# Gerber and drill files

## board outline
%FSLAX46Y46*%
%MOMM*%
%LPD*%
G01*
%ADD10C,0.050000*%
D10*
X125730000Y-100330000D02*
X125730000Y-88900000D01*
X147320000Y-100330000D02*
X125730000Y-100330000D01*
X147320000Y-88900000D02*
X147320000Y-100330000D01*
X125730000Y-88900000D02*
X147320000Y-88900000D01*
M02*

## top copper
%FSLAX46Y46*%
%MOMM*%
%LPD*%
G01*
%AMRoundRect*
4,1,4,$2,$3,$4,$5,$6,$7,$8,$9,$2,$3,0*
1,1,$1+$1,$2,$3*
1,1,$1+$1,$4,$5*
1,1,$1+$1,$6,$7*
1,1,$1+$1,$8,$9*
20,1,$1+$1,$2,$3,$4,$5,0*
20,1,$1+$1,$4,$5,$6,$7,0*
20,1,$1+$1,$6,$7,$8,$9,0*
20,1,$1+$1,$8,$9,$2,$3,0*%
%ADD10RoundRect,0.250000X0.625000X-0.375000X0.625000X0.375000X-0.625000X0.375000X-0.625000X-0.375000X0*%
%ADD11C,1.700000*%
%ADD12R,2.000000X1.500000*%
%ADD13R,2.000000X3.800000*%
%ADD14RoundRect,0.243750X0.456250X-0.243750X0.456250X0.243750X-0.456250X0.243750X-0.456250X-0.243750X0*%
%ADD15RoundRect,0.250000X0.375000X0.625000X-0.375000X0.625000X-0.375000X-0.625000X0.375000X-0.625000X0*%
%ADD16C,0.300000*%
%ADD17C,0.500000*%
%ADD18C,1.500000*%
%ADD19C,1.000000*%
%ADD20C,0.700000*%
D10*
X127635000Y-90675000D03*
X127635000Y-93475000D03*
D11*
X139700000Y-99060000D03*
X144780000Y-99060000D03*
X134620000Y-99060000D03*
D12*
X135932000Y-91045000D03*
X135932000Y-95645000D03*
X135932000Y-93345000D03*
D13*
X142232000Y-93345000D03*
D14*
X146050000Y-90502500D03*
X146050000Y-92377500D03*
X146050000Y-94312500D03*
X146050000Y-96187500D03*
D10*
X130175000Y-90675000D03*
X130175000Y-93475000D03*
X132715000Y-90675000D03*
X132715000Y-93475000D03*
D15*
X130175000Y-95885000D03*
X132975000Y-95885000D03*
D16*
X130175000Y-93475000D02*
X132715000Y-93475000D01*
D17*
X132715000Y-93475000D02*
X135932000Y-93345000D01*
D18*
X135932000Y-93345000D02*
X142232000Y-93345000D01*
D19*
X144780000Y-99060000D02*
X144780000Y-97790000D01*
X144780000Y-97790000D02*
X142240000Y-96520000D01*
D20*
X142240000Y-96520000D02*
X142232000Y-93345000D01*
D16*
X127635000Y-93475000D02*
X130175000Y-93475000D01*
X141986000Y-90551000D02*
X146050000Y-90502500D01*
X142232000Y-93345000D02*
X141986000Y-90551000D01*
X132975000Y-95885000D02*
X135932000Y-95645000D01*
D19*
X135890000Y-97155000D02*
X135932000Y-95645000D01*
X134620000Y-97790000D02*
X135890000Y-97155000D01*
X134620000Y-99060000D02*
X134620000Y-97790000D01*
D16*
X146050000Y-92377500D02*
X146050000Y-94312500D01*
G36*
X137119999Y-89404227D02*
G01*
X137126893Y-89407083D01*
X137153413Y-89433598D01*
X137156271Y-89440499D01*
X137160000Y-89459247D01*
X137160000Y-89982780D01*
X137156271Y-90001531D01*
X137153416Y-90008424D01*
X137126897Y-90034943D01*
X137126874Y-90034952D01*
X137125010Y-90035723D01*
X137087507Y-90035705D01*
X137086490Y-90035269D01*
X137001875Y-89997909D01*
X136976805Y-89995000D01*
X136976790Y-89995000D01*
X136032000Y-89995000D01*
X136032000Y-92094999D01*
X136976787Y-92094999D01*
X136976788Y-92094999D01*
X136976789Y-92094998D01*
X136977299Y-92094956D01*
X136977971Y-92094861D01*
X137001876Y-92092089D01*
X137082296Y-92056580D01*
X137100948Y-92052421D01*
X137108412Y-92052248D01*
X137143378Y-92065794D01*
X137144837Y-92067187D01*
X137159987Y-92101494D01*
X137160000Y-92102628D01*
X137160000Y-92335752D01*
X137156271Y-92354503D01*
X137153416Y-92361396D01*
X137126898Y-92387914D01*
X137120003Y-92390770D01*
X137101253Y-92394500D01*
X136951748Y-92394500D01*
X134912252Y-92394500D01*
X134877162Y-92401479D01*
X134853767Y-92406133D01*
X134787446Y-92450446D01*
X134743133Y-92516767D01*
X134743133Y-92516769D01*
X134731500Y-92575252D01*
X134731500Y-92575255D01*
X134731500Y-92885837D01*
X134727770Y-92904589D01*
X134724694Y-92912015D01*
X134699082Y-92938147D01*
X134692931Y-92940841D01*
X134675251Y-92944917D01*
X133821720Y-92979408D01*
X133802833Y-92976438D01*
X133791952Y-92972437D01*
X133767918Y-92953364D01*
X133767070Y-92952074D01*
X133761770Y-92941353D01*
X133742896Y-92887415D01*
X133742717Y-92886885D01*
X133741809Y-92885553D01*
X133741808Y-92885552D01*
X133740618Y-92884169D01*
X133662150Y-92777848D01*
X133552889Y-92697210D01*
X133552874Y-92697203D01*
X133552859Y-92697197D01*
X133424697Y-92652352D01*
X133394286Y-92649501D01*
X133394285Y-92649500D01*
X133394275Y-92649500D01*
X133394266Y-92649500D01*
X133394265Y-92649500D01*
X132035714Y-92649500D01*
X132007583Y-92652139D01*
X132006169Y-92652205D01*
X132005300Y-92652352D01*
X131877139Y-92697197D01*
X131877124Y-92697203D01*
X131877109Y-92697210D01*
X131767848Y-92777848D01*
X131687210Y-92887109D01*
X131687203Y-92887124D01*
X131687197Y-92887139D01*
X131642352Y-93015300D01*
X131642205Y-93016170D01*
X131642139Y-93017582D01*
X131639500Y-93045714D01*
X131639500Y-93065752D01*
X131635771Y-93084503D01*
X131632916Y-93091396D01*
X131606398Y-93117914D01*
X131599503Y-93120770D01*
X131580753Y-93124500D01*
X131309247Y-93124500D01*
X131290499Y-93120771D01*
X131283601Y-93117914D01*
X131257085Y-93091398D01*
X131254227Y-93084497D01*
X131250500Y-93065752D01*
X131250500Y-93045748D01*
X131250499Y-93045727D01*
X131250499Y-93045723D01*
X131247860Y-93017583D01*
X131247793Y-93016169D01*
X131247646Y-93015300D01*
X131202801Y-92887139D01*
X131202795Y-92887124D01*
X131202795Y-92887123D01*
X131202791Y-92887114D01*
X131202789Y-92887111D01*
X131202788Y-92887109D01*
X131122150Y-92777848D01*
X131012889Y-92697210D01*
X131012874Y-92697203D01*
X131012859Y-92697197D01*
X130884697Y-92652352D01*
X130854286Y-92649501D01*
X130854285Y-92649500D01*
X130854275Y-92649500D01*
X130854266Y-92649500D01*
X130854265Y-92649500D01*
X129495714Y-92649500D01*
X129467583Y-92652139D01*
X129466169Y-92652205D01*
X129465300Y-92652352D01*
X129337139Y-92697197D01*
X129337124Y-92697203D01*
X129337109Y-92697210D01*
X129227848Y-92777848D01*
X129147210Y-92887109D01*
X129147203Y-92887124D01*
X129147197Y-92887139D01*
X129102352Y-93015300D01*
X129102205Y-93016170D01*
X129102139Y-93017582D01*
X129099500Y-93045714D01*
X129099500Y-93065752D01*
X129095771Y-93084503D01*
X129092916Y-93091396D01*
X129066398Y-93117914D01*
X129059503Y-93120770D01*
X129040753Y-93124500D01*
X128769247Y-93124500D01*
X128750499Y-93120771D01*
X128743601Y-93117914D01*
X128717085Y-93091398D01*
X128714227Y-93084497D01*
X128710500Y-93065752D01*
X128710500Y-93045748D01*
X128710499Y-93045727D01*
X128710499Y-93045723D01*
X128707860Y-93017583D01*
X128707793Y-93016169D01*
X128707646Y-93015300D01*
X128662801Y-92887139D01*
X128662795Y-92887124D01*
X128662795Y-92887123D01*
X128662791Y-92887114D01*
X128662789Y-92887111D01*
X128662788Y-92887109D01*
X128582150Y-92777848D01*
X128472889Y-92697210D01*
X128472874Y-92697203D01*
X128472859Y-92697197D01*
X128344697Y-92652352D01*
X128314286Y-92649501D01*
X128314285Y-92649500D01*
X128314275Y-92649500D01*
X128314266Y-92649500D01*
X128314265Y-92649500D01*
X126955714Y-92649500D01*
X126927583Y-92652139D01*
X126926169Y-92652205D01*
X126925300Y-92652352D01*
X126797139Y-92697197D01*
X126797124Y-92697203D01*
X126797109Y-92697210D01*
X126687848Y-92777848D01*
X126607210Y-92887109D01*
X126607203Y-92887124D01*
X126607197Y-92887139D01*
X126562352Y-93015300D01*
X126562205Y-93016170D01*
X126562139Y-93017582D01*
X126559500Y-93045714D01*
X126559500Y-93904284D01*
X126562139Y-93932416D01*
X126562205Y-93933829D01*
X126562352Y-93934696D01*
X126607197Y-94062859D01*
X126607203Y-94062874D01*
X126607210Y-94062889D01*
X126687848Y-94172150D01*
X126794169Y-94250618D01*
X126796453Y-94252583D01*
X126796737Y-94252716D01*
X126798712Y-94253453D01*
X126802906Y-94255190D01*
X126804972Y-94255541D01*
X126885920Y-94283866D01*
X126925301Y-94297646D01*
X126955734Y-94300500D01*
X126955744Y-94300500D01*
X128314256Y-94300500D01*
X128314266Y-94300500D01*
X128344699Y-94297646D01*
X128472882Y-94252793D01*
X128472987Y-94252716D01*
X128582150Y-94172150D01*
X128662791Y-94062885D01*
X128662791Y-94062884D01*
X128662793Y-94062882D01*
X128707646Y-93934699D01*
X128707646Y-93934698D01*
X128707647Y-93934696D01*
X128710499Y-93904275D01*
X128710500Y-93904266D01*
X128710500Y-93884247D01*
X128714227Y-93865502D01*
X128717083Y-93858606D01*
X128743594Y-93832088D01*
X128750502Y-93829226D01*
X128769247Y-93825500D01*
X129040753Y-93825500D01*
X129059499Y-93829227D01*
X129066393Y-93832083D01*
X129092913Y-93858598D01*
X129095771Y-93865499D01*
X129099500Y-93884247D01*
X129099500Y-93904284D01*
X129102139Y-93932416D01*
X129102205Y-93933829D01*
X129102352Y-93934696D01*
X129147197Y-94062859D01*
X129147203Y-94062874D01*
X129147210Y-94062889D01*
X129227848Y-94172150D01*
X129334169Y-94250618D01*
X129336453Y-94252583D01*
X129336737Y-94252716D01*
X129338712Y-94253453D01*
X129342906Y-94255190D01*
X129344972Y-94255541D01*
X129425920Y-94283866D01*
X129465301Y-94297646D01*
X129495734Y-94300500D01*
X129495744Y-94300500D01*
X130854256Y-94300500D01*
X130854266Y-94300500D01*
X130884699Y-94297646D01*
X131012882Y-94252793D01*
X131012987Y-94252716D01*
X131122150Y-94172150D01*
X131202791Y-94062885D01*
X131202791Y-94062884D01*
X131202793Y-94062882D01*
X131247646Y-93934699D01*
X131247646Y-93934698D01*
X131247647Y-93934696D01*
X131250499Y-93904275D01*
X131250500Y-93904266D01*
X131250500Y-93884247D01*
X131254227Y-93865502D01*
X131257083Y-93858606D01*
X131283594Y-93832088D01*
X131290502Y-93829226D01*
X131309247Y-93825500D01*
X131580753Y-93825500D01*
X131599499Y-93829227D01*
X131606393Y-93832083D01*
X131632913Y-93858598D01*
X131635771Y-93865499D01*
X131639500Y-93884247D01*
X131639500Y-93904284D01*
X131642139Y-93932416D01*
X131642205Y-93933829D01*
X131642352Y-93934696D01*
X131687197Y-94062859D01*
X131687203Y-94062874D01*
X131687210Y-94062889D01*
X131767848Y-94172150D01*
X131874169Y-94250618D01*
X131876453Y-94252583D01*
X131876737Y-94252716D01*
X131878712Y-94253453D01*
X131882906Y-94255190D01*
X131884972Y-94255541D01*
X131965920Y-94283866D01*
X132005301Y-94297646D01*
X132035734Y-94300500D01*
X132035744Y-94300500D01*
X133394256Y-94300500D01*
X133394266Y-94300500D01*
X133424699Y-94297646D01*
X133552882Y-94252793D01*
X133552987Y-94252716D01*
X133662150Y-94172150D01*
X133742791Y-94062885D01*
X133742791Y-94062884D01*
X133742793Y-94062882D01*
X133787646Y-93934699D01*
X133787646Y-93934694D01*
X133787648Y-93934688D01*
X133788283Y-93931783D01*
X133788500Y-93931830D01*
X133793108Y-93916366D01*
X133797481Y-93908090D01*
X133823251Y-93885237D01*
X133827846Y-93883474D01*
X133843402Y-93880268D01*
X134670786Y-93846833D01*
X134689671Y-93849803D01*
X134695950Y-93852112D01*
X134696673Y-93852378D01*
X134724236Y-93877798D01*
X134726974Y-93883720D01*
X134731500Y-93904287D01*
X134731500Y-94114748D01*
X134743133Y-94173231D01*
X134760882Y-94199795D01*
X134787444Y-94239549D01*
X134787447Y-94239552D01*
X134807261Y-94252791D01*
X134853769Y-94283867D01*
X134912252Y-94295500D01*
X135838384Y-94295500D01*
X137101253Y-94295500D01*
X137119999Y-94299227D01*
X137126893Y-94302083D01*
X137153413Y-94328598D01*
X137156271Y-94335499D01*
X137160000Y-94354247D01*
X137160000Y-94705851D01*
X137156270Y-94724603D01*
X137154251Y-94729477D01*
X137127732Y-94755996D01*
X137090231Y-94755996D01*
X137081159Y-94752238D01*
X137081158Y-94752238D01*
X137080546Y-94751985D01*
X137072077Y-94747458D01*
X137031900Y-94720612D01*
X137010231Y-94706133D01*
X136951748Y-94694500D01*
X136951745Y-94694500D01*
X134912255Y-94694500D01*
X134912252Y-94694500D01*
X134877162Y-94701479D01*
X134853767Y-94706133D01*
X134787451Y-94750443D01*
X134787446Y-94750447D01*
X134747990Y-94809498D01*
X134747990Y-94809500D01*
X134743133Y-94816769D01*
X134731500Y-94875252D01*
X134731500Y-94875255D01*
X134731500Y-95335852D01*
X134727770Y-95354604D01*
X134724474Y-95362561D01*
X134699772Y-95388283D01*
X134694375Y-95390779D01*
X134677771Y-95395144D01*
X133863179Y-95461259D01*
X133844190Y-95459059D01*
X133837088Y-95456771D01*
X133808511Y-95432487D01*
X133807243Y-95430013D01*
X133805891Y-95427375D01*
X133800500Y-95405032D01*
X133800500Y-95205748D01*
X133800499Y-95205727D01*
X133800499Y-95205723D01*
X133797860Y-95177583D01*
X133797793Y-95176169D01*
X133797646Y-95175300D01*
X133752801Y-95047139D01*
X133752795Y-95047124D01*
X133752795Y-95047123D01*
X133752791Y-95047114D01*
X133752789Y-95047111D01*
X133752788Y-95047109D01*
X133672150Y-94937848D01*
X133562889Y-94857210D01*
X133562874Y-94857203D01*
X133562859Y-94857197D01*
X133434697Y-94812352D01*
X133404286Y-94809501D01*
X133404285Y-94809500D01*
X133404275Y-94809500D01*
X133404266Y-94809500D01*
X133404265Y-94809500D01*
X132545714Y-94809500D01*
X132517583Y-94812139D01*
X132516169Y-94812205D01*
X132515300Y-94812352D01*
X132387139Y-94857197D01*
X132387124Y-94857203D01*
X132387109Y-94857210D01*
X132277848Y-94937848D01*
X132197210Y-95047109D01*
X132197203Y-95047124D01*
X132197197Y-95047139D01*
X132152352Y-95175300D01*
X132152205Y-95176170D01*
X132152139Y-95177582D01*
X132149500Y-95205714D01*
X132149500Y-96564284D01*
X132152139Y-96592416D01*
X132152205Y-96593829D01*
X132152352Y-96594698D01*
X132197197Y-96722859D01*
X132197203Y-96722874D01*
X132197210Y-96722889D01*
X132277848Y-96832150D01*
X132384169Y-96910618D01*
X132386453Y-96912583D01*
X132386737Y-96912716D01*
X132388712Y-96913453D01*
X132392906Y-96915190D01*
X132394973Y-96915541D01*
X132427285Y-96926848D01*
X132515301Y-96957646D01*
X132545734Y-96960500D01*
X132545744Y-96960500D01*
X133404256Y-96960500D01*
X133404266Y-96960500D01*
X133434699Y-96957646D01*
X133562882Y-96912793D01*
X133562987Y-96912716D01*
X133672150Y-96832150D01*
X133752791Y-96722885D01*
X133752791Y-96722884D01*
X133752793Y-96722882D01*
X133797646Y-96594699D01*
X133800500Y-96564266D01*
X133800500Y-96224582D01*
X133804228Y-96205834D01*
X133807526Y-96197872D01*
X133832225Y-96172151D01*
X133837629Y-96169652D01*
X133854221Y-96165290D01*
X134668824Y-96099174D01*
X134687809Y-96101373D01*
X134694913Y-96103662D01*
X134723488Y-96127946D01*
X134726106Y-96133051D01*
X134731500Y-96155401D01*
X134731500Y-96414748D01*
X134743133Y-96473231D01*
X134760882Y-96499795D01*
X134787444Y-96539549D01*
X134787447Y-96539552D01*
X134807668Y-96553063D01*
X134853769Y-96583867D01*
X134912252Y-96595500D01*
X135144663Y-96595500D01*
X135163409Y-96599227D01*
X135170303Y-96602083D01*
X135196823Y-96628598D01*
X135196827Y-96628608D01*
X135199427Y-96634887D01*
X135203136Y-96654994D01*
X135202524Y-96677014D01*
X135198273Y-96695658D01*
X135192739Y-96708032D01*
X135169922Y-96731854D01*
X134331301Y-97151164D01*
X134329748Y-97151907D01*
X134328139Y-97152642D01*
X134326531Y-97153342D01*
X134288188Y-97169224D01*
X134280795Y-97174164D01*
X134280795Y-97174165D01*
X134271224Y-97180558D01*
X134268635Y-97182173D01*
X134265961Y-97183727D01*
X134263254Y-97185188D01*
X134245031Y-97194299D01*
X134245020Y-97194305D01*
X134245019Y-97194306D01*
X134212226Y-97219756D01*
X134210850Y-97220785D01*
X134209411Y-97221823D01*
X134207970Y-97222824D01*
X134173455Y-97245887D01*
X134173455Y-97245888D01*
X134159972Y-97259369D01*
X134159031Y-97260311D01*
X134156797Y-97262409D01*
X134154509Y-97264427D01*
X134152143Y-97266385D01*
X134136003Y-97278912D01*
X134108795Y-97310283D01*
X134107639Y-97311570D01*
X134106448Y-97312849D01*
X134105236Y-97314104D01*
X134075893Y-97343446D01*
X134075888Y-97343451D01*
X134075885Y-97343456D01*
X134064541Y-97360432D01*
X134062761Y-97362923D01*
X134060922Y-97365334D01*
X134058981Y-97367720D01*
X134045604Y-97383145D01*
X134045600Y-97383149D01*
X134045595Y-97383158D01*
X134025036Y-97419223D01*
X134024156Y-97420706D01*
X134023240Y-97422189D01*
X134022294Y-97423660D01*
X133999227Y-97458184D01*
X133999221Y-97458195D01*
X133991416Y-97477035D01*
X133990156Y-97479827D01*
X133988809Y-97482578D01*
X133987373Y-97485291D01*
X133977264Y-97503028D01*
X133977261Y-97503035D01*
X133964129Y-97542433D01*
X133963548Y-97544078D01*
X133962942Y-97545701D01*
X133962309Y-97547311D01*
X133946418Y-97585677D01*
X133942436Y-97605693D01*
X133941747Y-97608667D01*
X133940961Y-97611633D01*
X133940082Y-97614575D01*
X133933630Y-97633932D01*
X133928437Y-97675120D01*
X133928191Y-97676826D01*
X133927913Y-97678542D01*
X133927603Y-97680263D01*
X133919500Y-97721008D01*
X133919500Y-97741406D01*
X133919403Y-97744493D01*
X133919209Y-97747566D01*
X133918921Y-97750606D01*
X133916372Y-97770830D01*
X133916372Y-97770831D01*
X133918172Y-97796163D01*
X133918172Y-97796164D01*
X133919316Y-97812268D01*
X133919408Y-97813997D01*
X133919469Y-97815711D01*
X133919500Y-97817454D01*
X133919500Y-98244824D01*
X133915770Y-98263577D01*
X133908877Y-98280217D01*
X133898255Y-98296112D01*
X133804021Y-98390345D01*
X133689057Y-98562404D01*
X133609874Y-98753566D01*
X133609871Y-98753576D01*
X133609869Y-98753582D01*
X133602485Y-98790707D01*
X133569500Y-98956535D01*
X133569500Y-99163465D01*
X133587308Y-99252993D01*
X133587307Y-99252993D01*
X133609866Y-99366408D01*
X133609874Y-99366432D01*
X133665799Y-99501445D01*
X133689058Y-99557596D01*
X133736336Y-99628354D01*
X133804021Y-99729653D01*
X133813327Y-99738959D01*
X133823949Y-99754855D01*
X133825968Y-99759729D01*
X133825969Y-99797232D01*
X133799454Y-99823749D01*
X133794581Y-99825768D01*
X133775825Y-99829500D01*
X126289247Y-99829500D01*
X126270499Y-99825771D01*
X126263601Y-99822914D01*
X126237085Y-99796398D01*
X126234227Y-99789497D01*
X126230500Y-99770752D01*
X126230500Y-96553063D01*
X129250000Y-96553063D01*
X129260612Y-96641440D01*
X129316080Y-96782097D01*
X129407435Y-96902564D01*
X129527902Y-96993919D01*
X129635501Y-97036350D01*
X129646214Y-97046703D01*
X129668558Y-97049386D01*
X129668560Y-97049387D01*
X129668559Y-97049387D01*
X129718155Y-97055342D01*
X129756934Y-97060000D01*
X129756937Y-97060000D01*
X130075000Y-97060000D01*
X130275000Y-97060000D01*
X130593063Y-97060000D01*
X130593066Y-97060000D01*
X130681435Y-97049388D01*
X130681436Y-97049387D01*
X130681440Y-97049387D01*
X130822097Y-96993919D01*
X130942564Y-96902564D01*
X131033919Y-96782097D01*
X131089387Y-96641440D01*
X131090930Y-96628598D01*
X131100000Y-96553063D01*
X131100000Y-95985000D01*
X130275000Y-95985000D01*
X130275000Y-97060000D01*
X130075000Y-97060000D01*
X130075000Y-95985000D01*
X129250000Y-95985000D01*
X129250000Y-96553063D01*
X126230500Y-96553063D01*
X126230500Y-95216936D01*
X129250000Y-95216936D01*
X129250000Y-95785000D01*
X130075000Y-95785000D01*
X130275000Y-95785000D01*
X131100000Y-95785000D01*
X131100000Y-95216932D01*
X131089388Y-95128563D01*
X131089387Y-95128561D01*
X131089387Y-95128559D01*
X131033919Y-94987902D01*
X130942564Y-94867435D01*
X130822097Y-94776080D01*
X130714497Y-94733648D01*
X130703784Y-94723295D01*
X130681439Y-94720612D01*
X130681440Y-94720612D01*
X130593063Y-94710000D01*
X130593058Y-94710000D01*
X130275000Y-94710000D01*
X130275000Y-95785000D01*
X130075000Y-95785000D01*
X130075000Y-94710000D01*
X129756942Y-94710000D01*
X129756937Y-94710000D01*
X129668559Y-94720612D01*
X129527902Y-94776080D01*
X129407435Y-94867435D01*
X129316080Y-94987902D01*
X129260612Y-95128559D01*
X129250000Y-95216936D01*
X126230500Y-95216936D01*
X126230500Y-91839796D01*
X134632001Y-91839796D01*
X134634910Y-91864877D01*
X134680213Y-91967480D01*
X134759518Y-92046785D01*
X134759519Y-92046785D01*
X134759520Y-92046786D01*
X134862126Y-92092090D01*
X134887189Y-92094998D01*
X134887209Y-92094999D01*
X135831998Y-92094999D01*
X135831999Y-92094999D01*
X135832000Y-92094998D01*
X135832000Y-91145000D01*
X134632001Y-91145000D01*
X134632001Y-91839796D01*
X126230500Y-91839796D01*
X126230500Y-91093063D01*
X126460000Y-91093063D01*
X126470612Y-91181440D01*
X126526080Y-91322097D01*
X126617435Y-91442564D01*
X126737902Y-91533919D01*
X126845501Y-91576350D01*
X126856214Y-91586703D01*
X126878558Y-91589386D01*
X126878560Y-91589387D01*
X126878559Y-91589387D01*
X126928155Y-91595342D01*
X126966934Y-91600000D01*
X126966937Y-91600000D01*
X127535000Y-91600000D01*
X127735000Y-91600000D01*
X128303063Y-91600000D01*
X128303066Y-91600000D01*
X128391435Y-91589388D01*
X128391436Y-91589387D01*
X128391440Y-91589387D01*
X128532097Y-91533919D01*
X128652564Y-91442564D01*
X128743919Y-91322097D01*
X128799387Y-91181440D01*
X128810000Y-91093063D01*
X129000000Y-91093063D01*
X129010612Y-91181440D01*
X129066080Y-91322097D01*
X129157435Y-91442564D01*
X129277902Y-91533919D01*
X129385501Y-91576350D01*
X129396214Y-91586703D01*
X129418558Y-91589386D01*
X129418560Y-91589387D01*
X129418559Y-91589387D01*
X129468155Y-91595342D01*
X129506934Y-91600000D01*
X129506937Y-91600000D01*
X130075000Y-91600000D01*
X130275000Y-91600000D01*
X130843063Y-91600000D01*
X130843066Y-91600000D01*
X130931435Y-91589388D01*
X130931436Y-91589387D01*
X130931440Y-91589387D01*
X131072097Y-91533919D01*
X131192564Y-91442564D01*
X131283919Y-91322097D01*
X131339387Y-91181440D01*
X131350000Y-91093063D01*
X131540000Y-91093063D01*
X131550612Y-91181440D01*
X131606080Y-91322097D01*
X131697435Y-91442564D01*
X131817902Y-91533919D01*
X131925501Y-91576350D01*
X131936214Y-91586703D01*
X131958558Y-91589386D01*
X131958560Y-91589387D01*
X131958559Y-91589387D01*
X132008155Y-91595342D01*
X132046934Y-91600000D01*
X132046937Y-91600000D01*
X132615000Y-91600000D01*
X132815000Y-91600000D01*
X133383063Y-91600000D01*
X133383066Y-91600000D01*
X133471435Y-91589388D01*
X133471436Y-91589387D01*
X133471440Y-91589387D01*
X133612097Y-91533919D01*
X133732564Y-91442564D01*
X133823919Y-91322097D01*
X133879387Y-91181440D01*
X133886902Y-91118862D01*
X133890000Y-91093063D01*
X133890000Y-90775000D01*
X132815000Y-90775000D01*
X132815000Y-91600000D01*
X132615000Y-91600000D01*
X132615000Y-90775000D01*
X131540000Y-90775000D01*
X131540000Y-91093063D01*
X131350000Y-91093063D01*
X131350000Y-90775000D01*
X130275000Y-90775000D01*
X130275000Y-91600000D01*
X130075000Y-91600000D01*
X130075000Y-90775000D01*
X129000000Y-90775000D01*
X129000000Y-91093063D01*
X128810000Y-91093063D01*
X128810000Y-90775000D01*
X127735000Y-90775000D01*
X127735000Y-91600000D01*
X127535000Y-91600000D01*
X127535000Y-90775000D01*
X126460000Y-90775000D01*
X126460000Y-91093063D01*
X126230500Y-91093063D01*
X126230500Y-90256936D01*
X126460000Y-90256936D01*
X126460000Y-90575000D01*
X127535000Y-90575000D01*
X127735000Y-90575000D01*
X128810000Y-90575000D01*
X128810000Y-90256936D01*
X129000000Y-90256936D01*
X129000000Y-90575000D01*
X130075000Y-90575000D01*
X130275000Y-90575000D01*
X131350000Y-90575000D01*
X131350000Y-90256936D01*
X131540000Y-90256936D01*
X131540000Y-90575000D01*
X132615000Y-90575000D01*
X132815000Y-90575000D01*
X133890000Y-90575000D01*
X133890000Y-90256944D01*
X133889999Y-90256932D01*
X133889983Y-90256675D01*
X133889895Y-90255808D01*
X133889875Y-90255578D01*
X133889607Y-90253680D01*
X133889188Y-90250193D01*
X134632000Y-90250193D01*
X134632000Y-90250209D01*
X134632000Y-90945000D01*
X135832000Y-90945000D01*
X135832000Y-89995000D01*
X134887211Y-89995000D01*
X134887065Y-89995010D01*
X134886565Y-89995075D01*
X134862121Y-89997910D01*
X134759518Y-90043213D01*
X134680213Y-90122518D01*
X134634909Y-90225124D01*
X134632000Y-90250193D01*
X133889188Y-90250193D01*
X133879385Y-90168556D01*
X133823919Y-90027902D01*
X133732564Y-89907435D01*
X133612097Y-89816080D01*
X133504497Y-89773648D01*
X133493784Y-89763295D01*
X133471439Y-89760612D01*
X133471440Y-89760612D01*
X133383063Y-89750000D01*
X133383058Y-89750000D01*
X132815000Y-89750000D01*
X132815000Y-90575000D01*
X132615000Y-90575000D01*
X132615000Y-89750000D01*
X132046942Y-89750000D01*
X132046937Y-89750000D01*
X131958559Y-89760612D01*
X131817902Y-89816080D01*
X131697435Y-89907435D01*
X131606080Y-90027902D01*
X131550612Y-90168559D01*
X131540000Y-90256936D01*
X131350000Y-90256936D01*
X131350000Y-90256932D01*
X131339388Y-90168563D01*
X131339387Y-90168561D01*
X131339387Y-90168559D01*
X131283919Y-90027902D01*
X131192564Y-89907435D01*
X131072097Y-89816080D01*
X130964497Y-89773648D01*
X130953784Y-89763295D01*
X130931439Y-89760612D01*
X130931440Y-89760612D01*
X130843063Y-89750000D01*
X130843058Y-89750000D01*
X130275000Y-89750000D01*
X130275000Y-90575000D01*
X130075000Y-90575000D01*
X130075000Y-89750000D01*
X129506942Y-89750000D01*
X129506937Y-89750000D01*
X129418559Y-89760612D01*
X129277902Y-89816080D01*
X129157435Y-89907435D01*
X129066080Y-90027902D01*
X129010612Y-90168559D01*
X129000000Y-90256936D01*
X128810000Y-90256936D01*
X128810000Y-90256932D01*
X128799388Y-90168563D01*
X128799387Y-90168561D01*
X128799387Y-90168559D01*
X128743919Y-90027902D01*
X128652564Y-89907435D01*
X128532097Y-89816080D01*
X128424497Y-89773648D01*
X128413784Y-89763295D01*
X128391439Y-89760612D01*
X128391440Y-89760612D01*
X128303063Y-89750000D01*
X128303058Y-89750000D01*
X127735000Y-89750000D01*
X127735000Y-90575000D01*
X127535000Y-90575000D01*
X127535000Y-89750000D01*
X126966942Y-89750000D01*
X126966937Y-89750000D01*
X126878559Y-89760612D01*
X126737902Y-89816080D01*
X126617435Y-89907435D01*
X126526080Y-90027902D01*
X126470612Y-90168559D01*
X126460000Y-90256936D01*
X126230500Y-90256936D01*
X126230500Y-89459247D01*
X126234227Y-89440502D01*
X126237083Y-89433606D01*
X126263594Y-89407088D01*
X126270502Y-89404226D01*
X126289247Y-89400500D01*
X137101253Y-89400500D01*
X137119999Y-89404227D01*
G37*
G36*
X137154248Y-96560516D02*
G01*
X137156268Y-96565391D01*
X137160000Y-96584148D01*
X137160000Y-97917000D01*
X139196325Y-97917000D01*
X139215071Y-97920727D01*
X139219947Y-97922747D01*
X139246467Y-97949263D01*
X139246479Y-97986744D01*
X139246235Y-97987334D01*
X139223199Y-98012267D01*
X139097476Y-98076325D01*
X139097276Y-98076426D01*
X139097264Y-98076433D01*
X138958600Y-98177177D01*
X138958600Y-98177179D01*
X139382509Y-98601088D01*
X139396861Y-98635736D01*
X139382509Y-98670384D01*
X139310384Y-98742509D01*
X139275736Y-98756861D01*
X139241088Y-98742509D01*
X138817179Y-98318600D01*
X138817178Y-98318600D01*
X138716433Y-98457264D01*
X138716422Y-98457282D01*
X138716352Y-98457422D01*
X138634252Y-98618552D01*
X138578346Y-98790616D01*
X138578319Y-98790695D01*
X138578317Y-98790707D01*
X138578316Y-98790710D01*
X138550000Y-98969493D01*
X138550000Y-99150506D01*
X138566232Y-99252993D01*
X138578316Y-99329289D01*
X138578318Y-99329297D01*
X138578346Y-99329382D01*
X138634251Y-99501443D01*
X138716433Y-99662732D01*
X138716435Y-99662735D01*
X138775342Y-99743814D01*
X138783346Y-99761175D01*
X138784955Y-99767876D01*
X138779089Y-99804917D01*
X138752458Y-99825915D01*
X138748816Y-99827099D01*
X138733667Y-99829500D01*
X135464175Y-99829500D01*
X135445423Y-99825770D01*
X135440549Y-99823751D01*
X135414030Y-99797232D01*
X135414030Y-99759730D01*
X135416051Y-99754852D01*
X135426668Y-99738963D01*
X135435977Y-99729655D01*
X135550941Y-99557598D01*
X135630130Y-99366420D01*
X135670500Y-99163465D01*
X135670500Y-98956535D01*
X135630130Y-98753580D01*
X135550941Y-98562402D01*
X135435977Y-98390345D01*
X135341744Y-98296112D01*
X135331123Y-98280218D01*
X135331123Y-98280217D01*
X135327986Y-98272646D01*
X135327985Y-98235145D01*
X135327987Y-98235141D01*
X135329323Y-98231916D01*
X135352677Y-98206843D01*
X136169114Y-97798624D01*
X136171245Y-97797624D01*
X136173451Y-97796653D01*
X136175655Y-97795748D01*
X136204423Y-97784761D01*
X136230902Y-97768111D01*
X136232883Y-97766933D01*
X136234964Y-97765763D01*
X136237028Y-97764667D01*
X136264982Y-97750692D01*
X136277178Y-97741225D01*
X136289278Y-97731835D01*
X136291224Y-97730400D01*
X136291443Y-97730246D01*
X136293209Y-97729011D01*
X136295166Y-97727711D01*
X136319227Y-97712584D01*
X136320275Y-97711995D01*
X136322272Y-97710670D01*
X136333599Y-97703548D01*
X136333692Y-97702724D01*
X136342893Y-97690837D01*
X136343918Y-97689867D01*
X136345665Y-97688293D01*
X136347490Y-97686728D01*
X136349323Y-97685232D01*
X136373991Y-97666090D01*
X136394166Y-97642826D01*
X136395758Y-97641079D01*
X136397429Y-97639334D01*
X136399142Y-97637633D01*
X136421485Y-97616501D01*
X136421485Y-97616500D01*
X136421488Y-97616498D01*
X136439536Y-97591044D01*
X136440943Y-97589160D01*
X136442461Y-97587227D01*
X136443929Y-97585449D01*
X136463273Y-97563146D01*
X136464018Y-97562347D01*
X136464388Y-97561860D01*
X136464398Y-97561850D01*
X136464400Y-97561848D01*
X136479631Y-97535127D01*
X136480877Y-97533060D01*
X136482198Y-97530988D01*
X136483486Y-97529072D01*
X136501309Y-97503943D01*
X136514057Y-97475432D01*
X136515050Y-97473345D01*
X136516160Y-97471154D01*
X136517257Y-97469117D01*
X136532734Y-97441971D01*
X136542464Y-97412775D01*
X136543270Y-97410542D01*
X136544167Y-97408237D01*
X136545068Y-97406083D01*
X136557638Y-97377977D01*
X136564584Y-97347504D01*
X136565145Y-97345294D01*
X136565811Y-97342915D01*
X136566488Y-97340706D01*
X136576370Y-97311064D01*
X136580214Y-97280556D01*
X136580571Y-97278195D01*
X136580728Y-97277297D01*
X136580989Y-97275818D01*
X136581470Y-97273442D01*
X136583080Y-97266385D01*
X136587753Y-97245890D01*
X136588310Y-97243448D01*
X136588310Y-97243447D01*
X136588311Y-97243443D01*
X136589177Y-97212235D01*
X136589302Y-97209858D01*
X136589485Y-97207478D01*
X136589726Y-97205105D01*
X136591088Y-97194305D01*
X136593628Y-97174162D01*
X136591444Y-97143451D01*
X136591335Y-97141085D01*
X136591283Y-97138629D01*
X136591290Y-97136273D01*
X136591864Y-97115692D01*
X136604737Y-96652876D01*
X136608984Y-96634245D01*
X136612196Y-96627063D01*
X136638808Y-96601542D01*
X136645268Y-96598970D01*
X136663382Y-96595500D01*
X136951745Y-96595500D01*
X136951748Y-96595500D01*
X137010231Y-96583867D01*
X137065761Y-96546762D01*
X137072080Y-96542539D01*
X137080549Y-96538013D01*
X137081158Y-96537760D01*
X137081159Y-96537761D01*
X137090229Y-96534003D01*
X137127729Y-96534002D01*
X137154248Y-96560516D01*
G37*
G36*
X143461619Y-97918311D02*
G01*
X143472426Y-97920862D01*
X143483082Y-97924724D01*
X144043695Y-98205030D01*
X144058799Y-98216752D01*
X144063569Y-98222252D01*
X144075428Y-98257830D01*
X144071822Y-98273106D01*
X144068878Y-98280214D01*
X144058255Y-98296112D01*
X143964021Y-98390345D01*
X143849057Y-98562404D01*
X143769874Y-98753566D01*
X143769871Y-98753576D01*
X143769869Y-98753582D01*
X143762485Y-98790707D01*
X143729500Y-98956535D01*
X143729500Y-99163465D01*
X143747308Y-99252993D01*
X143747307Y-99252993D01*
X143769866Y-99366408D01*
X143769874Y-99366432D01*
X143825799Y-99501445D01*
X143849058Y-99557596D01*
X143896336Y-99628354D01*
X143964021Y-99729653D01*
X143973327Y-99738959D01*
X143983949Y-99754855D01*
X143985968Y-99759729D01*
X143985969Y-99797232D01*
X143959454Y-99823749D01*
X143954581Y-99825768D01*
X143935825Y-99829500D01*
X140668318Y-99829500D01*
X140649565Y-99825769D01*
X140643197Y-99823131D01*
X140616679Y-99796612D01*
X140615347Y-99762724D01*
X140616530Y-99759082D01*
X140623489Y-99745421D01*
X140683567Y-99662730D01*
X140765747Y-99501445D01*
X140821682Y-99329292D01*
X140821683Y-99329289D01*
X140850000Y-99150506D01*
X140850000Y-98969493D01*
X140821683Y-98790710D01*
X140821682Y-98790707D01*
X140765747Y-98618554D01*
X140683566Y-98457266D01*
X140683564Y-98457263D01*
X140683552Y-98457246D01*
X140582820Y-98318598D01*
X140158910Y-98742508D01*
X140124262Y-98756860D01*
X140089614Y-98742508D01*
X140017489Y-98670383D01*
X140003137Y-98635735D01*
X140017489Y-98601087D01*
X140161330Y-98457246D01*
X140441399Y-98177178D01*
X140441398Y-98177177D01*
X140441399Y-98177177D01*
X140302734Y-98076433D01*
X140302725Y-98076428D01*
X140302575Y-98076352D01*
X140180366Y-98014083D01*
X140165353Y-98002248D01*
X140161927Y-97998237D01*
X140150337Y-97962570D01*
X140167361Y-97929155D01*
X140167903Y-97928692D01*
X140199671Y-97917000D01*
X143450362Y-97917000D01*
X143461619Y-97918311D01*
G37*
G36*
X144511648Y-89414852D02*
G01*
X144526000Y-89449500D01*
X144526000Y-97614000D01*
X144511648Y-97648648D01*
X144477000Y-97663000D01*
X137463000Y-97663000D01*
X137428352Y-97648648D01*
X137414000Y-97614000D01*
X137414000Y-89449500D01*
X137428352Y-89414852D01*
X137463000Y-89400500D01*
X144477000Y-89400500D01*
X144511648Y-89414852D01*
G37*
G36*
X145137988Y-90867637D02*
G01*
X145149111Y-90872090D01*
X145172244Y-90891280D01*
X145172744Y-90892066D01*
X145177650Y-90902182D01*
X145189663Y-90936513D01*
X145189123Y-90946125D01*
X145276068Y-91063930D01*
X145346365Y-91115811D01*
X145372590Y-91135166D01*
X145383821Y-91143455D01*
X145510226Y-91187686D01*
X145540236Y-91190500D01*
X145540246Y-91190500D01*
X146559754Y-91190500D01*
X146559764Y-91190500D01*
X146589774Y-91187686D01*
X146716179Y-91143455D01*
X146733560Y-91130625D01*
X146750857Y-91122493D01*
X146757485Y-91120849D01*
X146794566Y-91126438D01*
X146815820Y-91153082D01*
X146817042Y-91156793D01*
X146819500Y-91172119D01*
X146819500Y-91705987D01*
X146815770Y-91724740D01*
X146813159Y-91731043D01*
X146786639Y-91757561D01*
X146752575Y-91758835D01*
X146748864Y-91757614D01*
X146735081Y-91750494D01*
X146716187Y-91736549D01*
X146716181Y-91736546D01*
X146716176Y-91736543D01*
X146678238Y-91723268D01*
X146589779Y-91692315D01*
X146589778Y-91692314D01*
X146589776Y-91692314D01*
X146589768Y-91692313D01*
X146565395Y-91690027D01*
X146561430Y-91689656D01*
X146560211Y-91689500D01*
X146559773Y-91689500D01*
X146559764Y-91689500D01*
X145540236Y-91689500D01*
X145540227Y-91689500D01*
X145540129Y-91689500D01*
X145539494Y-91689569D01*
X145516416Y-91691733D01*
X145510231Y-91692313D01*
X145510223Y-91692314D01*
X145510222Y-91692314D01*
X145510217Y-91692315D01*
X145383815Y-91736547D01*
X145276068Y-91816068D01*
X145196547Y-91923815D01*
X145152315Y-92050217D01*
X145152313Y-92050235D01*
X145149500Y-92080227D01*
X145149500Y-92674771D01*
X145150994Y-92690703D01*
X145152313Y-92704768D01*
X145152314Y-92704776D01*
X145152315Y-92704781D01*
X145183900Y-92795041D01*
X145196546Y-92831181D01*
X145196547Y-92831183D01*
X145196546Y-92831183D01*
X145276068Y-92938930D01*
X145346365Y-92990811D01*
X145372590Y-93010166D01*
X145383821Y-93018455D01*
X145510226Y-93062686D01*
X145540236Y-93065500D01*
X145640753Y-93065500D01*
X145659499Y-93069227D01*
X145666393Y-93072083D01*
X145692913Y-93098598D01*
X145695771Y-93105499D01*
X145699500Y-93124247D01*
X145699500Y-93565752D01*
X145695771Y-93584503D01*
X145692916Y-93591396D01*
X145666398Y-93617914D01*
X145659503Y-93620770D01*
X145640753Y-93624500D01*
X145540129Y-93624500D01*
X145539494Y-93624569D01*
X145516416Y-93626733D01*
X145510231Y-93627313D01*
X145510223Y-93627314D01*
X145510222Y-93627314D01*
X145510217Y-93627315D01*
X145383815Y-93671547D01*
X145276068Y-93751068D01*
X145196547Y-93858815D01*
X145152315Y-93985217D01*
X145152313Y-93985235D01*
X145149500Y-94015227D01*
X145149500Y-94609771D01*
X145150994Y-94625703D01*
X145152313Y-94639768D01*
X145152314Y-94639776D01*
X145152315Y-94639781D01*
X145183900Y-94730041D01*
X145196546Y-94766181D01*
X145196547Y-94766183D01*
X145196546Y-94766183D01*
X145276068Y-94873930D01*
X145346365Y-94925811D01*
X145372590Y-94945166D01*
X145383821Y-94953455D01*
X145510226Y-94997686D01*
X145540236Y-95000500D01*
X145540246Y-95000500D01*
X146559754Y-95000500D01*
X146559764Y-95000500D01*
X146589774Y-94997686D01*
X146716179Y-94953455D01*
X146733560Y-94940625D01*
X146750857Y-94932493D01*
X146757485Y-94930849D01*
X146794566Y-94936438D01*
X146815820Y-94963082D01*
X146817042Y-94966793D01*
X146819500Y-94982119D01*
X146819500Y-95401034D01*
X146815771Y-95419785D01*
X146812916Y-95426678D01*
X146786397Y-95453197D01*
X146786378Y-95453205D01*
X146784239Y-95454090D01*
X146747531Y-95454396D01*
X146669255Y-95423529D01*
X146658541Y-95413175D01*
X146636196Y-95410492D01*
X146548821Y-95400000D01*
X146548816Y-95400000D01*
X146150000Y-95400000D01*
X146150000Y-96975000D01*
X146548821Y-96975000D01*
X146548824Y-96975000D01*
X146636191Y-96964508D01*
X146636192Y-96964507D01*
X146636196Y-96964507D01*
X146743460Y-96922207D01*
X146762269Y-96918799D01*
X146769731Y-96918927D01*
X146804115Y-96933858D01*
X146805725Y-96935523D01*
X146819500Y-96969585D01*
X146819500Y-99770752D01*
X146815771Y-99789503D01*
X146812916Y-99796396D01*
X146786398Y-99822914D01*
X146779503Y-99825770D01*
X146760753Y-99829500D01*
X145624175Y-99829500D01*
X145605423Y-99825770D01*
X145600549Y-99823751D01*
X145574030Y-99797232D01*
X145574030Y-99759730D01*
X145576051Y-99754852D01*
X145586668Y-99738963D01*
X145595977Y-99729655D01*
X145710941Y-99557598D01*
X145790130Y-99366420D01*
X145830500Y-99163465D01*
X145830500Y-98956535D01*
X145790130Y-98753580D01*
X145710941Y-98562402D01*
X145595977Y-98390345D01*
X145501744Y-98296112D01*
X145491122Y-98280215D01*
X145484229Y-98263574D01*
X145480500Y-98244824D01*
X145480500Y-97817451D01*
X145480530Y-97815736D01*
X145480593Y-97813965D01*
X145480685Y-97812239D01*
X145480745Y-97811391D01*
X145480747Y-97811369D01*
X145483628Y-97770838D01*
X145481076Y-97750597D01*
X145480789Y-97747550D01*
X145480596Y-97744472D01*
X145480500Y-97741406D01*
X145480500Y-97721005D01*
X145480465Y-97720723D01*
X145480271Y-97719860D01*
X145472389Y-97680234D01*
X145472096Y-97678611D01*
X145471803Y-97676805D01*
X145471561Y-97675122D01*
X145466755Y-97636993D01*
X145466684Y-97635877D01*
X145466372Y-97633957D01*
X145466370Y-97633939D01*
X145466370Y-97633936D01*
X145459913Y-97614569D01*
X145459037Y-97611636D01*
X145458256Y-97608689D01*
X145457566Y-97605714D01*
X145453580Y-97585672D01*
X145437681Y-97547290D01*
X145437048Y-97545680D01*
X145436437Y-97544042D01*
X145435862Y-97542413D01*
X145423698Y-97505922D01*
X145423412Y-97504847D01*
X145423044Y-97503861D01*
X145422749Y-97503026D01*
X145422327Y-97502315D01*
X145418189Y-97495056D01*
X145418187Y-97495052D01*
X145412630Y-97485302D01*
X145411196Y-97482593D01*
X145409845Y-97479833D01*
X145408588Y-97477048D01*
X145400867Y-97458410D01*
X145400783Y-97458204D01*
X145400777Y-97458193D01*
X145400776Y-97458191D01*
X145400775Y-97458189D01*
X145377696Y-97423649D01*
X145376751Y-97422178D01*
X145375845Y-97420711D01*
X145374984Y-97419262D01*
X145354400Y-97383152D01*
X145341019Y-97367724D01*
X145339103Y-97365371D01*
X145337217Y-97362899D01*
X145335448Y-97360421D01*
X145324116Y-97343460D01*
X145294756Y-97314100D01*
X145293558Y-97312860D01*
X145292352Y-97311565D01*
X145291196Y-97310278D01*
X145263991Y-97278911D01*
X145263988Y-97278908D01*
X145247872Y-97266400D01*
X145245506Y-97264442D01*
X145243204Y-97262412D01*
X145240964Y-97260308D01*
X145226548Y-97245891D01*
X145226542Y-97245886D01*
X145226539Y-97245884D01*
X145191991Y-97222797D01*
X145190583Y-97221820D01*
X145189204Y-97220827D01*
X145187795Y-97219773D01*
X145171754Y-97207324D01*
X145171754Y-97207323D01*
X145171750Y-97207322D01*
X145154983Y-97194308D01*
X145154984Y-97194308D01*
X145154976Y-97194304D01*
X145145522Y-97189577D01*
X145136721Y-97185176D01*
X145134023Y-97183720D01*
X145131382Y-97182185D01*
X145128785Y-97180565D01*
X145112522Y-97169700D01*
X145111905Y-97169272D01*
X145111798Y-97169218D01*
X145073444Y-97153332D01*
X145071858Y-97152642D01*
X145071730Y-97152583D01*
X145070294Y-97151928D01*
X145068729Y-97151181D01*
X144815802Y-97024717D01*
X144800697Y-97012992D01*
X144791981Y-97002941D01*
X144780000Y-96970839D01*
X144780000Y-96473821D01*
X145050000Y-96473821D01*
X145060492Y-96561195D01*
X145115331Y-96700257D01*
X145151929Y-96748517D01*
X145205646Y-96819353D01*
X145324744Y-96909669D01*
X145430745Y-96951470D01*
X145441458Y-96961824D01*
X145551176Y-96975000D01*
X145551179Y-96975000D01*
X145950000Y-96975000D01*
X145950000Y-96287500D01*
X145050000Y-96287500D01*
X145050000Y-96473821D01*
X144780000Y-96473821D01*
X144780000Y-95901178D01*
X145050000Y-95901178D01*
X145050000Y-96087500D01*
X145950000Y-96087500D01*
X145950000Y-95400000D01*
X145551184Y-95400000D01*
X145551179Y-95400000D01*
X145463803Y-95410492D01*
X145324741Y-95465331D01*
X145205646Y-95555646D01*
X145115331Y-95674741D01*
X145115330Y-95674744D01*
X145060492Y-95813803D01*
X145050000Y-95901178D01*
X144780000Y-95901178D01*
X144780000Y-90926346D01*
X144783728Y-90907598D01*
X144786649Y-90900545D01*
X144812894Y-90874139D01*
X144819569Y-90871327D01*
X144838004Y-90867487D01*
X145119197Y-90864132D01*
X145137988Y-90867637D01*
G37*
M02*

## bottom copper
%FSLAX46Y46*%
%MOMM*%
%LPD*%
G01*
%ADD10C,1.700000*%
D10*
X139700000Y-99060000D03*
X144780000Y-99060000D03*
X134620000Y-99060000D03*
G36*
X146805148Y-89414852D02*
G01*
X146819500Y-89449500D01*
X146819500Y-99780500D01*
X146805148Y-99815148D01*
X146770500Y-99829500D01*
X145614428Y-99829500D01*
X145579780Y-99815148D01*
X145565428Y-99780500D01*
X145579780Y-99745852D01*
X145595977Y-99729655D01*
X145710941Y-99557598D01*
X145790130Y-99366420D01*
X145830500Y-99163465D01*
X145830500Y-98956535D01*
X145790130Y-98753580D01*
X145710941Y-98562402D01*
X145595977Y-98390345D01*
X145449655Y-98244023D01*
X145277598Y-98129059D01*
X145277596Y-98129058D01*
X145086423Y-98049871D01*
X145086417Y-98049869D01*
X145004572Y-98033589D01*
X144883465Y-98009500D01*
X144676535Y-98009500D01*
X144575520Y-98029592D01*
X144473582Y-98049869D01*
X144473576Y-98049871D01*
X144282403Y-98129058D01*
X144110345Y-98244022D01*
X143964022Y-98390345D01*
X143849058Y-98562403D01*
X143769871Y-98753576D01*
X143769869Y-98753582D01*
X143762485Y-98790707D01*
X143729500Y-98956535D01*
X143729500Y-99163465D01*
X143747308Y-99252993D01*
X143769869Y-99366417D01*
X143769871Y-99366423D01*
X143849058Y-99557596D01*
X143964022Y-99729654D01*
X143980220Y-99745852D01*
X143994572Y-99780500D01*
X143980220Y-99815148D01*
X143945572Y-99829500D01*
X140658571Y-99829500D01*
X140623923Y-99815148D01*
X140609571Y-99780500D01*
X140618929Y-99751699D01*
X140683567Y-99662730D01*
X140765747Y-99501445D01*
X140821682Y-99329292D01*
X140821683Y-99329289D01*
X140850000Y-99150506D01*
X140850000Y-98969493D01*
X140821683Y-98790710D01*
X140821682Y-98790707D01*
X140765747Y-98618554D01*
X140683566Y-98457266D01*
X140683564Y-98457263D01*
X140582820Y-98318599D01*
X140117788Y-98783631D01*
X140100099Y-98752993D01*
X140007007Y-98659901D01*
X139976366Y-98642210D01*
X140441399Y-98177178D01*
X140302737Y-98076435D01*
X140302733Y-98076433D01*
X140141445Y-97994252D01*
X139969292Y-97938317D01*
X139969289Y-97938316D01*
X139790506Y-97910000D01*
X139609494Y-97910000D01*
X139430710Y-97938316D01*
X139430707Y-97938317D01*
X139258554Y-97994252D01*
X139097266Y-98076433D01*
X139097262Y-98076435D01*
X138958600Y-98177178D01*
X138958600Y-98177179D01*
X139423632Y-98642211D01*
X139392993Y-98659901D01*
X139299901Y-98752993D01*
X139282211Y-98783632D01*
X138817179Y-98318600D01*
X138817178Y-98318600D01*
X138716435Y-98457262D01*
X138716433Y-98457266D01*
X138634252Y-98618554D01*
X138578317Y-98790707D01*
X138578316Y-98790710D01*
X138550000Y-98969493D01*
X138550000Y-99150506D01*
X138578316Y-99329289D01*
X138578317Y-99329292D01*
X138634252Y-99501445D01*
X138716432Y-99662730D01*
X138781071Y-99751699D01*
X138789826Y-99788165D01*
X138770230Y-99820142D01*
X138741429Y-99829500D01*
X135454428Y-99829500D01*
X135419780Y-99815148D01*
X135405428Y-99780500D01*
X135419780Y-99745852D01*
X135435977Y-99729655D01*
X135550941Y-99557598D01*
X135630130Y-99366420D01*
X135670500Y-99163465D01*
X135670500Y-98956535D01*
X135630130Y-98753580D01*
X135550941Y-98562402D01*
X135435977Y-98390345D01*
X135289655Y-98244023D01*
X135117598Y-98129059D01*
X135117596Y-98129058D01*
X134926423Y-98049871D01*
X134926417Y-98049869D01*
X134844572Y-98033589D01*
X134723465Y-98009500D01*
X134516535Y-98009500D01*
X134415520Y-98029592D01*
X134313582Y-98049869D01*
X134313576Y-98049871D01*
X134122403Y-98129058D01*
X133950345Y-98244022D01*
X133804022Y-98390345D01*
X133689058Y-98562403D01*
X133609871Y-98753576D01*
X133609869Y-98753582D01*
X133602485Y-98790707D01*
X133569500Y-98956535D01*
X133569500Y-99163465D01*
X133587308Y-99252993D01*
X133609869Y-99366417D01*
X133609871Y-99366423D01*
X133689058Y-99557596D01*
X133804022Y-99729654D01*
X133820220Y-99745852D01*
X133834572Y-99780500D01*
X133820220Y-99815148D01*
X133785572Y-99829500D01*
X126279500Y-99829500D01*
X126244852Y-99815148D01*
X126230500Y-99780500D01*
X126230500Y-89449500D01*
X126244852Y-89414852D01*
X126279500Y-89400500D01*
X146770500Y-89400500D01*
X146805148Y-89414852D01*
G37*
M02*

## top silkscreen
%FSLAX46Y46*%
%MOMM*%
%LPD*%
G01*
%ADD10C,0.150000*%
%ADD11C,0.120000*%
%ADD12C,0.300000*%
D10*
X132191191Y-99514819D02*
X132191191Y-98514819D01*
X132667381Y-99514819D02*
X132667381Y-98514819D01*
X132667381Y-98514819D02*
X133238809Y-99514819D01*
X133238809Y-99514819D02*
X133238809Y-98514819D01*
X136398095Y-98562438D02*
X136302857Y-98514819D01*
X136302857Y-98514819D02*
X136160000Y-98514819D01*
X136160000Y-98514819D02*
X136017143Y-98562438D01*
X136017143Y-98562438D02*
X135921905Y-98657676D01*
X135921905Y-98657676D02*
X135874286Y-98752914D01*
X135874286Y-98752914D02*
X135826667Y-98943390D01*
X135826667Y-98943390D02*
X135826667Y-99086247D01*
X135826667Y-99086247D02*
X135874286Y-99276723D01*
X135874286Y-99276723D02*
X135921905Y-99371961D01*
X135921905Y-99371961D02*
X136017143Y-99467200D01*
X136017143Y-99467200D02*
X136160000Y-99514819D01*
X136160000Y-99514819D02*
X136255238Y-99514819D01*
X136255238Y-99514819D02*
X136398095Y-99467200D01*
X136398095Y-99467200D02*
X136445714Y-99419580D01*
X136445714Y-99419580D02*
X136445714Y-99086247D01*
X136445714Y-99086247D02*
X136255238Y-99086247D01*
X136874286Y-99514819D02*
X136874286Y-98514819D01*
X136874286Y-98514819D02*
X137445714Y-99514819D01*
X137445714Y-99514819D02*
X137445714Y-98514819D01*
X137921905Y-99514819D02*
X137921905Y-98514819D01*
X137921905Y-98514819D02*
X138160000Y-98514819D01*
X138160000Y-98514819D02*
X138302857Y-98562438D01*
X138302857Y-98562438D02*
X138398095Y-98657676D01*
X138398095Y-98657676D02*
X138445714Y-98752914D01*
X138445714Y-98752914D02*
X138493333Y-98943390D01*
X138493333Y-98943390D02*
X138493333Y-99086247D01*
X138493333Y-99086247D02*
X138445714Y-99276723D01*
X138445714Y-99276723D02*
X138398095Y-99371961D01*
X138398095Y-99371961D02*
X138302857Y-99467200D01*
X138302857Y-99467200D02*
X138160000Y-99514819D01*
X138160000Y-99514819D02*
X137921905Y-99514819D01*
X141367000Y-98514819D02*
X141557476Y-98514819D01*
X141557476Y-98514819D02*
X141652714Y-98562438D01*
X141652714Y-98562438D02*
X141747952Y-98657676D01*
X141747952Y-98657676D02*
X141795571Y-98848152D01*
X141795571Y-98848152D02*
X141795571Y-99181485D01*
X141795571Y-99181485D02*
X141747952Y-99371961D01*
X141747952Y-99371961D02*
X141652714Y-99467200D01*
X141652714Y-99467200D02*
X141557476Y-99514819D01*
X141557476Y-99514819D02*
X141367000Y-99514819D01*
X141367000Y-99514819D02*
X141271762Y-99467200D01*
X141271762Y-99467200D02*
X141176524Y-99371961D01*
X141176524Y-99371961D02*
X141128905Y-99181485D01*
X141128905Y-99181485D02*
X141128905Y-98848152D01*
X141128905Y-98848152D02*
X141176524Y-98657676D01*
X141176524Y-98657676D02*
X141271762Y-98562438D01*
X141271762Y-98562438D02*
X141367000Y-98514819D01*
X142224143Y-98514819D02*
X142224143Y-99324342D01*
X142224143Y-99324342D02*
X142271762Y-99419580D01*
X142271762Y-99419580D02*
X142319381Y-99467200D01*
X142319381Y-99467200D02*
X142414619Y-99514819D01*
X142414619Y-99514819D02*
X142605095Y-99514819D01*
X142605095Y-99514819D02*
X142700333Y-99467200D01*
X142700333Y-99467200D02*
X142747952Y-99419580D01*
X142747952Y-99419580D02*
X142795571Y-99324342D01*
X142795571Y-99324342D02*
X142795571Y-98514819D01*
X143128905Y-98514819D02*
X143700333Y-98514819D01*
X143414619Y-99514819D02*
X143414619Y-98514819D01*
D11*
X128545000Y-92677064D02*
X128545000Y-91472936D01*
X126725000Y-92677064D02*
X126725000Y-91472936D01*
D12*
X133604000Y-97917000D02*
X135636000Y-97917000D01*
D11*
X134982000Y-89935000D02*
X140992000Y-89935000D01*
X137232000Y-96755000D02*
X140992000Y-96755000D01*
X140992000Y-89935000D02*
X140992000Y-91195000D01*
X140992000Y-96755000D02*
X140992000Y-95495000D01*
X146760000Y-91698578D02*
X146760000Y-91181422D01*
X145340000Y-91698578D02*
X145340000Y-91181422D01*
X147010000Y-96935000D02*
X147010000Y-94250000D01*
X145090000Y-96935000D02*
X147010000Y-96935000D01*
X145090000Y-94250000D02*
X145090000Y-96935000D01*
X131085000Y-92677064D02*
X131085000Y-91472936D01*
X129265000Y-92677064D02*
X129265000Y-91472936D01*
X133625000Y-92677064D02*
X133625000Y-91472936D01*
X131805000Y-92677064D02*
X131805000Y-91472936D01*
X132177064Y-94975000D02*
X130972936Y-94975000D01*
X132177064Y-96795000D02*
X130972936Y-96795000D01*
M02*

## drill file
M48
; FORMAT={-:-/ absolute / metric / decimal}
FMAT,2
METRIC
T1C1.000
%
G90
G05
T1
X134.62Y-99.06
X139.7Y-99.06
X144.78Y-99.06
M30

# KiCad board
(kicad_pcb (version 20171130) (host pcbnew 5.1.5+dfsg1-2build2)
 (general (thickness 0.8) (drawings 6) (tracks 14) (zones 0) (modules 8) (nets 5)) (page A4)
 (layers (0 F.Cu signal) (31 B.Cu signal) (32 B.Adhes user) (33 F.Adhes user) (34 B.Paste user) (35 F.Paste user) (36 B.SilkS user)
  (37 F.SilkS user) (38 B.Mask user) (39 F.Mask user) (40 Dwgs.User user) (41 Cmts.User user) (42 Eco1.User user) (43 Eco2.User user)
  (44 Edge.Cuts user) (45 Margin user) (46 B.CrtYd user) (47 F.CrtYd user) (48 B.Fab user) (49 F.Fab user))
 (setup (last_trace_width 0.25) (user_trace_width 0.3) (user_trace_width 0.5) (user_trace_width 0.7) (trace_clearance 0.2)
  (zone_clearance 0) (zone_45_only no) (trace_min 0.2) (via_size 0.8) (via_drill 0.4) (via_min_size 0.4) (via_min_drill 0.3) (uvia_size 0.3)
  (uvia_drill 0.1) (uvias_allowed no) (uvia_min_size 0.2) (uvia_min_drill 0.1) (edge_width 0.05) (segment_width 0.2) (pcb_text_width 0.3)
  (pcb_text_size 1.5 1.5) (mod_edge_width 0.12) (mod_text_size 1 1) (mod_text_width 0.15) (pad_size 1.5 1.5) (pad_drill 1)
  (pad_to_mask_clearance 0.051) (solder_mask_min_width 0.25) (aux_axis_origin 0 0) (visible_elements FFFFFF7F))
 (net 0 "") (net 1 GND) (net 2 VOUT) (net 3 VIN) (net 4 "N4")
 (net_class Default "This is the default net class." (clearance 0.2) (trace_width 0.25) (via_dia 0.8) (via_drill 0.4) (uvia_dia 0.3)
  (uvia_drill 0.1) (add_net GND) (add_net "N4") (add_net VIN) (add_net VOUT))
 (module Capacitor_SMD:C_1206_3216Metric (layer F.Cu) (at 127.635 92.075 90)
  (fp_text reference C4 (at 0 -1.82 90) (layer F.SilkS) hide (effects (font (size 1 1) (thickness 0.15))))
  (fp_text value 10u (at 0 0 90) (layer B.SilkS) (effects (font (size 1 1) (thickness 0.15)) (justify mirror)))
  (fp_line (start -0.602064 0.91) (end 0.602064 0.91) (layer F.SilkS) (width 0.12))
  (fp_line (start -0.602064 -0.91) (end 0.602064 -0.91) (layer F.SilkS) (width 0.12))
  (pad 2 smd roundrect (at 1.4 0 90) (size 1.25 1.75) (layers F.Cu F.Paste F.Mask) (roundrect_rratio 0.2) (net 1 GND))
  (pad 1 smd roundrect (at -1.4 0 90) (size 1.25 1.75) (layers F.Cu F.Paste F.Mask) (roundrect_rratio 0.2) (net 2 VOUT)))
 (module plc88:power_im (layer F.Cu) (at 128.27 88.9)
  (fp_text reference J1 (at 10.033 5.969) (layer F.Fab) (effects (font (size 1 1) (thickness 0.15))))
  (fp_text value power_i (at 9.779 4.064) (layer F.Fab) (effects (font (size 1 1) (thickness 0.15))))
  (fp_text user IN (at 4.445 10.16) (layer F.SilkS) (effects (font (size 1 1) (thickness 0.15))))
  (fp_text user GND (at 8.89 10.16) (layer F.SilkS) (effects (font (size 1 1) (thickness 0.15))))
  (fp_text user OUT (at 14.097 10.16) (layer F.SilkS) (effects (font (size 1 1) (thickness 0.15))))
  (fp_line (start 5.334 9.017) (end 7.366 9.017) (layer F.SilkS) (width 0.3))
  (pad 3 thru_hole circle (at 11.43 10.16) (size 1.7 1.7) (drill 1) (layers *.Cu *.Mask) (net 1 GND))
  (pad 2 thru_hole circle (at 16.51 10.16) (size 1.7 1.7) (drill 1) (layers *.Cu *.Mask) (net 2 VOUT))
  (pad 1 thru_hole circle (at 6.35 10.16) (size 1.7 1.7) (drill 1) (layers *.Cu *.Mask) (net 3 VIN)))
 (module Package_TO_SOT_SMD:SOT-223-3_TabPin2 (layer F.Cu) (at 139.082 93.345)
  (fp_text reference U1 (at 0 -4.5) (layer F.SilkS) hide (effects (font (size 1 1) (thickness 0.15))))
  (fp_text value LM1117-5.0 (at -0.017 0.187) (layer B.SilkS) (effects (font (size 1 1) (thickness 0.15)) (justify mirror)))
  (fp_line (start -4.1 -3.41) (end 1.91 -3.41) (layer F.SilkS) (width 0.12))
  (fp_line (start -1.85 3.41) (end 1.91 3.41) (layer F.SilkS) (width 0.12))
  (fp_line (start 1.91 -3.41) (end 1.91 -2.15) (layer F.SilkS) (width 0.12))
  (fp_line (start 1.91 3.41) (end 1.91 2.15) (layer F.SilkS) (width 0.12))
  (pad 1 smd rect (at -3.15 -2.3) (size 2 1.5) (layers F.Cu F.Paste F.Mask) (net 1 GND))
  (pad 3 smd rect (at -3.15 2.3) (size 2 1.5) (layers F.Cu F.Paste F.Mask) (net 3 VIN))
  (pad 2 smd rect (at -3.15 0) (size 2 1.5) (layers F.Cu F.Paste F.Mask) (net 2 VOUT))
  (pad 2 smd rect (at 3.15 0) (size 2 3.8) (layers F.Cu F.Paste F.Mask) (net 2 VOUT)))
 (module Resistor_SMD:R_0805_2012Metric (layer F.Cu) (at 146.05 91.44 90)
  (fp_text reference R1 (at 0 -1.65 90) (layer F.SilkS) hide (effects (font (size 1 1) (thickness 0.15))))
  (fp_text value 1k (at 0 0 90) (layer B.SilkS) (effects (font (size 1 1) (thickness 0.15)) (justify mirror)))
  (fp_line (start -0.258578 0.71) (end 0.258578 0.71) (layer F.SilkS) (width 0.12))
  (fp_line (start -0.258578 -0.71) (end 0.258578 -0.71) (layer F.SilkS) (width 0.12))
  (pad 2 smd roundrect (at 0.9375 0 90) (size 0.975 1.4) (layers F.Cu F.Paste F.Mask) (roundrect_rratio 0.25) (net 2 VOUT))
  (pad 1 smd roundrect (at -0.9375 0 90) (size 0.975 1.4) (layers F.Cu F.Paste F.Mask) (roundrect_rratio 0.25) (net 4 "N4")))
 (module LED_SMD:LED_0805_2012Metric (layer F.Cu) (at 146.05 95.25 90)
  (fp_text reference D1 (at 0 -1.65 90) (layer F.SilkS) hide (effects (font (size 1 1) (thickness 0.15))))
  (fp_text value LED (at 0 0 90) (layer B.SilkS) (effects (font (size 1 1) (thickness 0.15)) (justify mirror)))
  (fp_line (start -1.685 0.96) (end 1 0.96) (layer F.SilkS) (width 0.12))
  (fp_line (start -1.685 -0.96) (end -1.685 0.96) (layer F.SilkS) (width 0.12))
  (fp_line (start 1 -0.96) (end -1.685 -0.96) (layer F.SilkS) (width 0.12))
  (pad 2 smd roundrect (at 0.9375 0 90) (size 0.975 1.4) (layers F.Cu F.Paste F.Mask) (roundrect_rratio 0.25) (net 4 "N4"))
  (pad 1 smd roundrect (at -0.9375 0 90) (size 0.975 1.4) (layers F.Cu F.Paste F.Mask) (roundrect_rratio 0.25) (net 1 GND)))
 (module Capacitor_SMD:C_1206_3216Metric (layer F.Cu) (at 130.175 92.075 90)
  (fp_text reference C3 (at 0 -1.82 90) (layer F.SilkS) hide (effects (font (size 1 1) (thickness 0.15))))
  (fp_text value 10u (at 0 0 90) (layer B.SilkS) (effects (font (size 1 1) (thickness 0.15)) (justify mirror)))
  (fp_line (start -0.602064 0.91) (end 0.602064 0.91) (layer F.SilkS) (width 0.12))
  (fp_line (start -0.602064 -0.91) (end 0.602064 -0.91) (layer F.SilkS) (width 0.12))
  (pad 2 smd roundrect (at 1.4 0 90) (size 1.25 1.75) (layers F.Cu F.Paste F.Mask) (roundrect_rratio 0.2) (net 1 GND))
  (pad 1 smd roundrect (at -1.4 0 90) (size 1.25 1.75) (layers F.Cu F.Paste F.Mask) (roundrect_rratio 0.2) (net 2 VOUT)))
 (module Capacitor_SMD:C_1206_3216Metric (layer F.Cu) (at 132.715 92.075 90)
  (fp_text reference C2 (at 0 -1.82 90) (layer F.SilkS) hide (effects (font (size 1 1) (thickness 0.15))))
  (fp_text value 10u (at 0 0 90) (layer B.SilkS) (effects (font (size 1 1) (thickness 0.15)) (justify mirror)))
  (fp_line (start -0.602064 0.91) (end 0.602064 0.91) (layer F.SilkS) (width 0.12))
  (fp_line (start -0.602064 -0.91) (end 0.602064 -0.91) (layer F.SilkS) (width 0.12))
  (pad 2 smd roundrect (at 1.4 0 90) (size 1.25 1.75) (layers F.Cu F.Paste F.Mask) (roundrect_rratio 0.2) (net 1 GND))
  (pad 1 smd roundrect (at -1.4 0 90) (size 1.25 1.75) (layers F.Cu F.Paste F.Mask) (roundrect_rratio 0.2) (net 2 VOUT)))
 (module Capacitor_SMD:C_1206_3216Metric (layer F.Cu) (at 131.575 95.885 180)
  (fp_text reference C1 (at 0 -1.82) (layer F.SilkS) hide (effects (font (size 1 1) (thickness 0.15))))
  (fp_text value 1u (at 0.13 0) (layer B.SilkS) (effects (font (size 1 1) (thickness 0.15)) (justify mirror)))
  (fp_line (start -0.602064 0.91) (end 0.602064 0.91) (layer F.SilkS) (width 0.12))
  (fp_line (start -0.602064 -0.91) (end 0.602064 -0.91) (layer F.SilkS) (width 0.12))
  (pad 2 smd roundrect (at 1.4 0 180) (size 1.25 1.75) (layers F.Cu F.Paste F.Mask) (roundrect_rratio 0.2) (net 1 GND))
  (pad 1 smd roundrect (at -1.4 0 180) (size 1.25 1.75) (layers F.Cu F.Paste F.Mask) (roundrect_rratio 0.2) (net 3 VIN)))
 (gr_line (start 125.73 100.33) (end 125.73 88.9) (layer Edge.Cuts) (width 0.05))
 (gr_line (start 147.32 100.33) (end 125.73 100.33) (layer Edge.Cuts) (width 0.05))
 (gr_line (start 147.32 88.9) (end 147.32 100.33) (layer Edge.Cuts) (width 0.05))
 (gr_line (start 125.73 88.9) (end 147.32 88.9) (layer Edge.Cuts) (width 0.05))
 (segment (start 130.175 93.475) (end 132.715 93.475) (width 0.3) (layer F.Cu) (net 2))
 (segment (start 132.715 93.475) (end 135.932 93.345) (width 0.5) (layer F.Cu) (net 2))
 (segment (start 135.932 93.345) (end 142.232 93.345) (width 1.5) (layer F.Cu) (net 2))
 (segment (start 144.78 99.06) (end 144.78 97.79) (width 1) (layer F.Cu) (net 2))
 (segment (start 144.78 97.79) (end 142.24 96.52) (width 1) (layer F.Cu) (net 2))
 (segment (start 142.24 96.52) (end 142.232 93.345) (width 0.7) (layer F.Cu) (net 2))
 (segment (start 127.635 93.475) (end 130.175 93.475) (width 0.3) (layer F.Cu) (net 2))
 (segment (start 141.986 90.551) (end 146.05 90.5025) (width 0.3) (layer F.Cu) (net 2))
 (segment (start 142.232 93.345) (end 141.986 90.551) (width 0.3) (layer F.Cu) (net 2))
 (segment (start 132.975 95.885) (end 135.932 95.645) (width 0.3) (layer F.Cu) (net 3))
 (segment (start 135.89 97.155) (end 135.932 95.645) (width 1) (layer F.Cu) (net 3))
 (segment (start 134.62 97.79) (end 135.89 97.155) (width 1) (layer F.Cu) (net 3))
 (segment (start 134.62 99.06) (end 134.62 97.79) (width 1) (layer F.Cu) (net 3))
 (segment (start 146.05 92.3775) (end 146.05 94.3125) (width 0.3) (layer F.Cu) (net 4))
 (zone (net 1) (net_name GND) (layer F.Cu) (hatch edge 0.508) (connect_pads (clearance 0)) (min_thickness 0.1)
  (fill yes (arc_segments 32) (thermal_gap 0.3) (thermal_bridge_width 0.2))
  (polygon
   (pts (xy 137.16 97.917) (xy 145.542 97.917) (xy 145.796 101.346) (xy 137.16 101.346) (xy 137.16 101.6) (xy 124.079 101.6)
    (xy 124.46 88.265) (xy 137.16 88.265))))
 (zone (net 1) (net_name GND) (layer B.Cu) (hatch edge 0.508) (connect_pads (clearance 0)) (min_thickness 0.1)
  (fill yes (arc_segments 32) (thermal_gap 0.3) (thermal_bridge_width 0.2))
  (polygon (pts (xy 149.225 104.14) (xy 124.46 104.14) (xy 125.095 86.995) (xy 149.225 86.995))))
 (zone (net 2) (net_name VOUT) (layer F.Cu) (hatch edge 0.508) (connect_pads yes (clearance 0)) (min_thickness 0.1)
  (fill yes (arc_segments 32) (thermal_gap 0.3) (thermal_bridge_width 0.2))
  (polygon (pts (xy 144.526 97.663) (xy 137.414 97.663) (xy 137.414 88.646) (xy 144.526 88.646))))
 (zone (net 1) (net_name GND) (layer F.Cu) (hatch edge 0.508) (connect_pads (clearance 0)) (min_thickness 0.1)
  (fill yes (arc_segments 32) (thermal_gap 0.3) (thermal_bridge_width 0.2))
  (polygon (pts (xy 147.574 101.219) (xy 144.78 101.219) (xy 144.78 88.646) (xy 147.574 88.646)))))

